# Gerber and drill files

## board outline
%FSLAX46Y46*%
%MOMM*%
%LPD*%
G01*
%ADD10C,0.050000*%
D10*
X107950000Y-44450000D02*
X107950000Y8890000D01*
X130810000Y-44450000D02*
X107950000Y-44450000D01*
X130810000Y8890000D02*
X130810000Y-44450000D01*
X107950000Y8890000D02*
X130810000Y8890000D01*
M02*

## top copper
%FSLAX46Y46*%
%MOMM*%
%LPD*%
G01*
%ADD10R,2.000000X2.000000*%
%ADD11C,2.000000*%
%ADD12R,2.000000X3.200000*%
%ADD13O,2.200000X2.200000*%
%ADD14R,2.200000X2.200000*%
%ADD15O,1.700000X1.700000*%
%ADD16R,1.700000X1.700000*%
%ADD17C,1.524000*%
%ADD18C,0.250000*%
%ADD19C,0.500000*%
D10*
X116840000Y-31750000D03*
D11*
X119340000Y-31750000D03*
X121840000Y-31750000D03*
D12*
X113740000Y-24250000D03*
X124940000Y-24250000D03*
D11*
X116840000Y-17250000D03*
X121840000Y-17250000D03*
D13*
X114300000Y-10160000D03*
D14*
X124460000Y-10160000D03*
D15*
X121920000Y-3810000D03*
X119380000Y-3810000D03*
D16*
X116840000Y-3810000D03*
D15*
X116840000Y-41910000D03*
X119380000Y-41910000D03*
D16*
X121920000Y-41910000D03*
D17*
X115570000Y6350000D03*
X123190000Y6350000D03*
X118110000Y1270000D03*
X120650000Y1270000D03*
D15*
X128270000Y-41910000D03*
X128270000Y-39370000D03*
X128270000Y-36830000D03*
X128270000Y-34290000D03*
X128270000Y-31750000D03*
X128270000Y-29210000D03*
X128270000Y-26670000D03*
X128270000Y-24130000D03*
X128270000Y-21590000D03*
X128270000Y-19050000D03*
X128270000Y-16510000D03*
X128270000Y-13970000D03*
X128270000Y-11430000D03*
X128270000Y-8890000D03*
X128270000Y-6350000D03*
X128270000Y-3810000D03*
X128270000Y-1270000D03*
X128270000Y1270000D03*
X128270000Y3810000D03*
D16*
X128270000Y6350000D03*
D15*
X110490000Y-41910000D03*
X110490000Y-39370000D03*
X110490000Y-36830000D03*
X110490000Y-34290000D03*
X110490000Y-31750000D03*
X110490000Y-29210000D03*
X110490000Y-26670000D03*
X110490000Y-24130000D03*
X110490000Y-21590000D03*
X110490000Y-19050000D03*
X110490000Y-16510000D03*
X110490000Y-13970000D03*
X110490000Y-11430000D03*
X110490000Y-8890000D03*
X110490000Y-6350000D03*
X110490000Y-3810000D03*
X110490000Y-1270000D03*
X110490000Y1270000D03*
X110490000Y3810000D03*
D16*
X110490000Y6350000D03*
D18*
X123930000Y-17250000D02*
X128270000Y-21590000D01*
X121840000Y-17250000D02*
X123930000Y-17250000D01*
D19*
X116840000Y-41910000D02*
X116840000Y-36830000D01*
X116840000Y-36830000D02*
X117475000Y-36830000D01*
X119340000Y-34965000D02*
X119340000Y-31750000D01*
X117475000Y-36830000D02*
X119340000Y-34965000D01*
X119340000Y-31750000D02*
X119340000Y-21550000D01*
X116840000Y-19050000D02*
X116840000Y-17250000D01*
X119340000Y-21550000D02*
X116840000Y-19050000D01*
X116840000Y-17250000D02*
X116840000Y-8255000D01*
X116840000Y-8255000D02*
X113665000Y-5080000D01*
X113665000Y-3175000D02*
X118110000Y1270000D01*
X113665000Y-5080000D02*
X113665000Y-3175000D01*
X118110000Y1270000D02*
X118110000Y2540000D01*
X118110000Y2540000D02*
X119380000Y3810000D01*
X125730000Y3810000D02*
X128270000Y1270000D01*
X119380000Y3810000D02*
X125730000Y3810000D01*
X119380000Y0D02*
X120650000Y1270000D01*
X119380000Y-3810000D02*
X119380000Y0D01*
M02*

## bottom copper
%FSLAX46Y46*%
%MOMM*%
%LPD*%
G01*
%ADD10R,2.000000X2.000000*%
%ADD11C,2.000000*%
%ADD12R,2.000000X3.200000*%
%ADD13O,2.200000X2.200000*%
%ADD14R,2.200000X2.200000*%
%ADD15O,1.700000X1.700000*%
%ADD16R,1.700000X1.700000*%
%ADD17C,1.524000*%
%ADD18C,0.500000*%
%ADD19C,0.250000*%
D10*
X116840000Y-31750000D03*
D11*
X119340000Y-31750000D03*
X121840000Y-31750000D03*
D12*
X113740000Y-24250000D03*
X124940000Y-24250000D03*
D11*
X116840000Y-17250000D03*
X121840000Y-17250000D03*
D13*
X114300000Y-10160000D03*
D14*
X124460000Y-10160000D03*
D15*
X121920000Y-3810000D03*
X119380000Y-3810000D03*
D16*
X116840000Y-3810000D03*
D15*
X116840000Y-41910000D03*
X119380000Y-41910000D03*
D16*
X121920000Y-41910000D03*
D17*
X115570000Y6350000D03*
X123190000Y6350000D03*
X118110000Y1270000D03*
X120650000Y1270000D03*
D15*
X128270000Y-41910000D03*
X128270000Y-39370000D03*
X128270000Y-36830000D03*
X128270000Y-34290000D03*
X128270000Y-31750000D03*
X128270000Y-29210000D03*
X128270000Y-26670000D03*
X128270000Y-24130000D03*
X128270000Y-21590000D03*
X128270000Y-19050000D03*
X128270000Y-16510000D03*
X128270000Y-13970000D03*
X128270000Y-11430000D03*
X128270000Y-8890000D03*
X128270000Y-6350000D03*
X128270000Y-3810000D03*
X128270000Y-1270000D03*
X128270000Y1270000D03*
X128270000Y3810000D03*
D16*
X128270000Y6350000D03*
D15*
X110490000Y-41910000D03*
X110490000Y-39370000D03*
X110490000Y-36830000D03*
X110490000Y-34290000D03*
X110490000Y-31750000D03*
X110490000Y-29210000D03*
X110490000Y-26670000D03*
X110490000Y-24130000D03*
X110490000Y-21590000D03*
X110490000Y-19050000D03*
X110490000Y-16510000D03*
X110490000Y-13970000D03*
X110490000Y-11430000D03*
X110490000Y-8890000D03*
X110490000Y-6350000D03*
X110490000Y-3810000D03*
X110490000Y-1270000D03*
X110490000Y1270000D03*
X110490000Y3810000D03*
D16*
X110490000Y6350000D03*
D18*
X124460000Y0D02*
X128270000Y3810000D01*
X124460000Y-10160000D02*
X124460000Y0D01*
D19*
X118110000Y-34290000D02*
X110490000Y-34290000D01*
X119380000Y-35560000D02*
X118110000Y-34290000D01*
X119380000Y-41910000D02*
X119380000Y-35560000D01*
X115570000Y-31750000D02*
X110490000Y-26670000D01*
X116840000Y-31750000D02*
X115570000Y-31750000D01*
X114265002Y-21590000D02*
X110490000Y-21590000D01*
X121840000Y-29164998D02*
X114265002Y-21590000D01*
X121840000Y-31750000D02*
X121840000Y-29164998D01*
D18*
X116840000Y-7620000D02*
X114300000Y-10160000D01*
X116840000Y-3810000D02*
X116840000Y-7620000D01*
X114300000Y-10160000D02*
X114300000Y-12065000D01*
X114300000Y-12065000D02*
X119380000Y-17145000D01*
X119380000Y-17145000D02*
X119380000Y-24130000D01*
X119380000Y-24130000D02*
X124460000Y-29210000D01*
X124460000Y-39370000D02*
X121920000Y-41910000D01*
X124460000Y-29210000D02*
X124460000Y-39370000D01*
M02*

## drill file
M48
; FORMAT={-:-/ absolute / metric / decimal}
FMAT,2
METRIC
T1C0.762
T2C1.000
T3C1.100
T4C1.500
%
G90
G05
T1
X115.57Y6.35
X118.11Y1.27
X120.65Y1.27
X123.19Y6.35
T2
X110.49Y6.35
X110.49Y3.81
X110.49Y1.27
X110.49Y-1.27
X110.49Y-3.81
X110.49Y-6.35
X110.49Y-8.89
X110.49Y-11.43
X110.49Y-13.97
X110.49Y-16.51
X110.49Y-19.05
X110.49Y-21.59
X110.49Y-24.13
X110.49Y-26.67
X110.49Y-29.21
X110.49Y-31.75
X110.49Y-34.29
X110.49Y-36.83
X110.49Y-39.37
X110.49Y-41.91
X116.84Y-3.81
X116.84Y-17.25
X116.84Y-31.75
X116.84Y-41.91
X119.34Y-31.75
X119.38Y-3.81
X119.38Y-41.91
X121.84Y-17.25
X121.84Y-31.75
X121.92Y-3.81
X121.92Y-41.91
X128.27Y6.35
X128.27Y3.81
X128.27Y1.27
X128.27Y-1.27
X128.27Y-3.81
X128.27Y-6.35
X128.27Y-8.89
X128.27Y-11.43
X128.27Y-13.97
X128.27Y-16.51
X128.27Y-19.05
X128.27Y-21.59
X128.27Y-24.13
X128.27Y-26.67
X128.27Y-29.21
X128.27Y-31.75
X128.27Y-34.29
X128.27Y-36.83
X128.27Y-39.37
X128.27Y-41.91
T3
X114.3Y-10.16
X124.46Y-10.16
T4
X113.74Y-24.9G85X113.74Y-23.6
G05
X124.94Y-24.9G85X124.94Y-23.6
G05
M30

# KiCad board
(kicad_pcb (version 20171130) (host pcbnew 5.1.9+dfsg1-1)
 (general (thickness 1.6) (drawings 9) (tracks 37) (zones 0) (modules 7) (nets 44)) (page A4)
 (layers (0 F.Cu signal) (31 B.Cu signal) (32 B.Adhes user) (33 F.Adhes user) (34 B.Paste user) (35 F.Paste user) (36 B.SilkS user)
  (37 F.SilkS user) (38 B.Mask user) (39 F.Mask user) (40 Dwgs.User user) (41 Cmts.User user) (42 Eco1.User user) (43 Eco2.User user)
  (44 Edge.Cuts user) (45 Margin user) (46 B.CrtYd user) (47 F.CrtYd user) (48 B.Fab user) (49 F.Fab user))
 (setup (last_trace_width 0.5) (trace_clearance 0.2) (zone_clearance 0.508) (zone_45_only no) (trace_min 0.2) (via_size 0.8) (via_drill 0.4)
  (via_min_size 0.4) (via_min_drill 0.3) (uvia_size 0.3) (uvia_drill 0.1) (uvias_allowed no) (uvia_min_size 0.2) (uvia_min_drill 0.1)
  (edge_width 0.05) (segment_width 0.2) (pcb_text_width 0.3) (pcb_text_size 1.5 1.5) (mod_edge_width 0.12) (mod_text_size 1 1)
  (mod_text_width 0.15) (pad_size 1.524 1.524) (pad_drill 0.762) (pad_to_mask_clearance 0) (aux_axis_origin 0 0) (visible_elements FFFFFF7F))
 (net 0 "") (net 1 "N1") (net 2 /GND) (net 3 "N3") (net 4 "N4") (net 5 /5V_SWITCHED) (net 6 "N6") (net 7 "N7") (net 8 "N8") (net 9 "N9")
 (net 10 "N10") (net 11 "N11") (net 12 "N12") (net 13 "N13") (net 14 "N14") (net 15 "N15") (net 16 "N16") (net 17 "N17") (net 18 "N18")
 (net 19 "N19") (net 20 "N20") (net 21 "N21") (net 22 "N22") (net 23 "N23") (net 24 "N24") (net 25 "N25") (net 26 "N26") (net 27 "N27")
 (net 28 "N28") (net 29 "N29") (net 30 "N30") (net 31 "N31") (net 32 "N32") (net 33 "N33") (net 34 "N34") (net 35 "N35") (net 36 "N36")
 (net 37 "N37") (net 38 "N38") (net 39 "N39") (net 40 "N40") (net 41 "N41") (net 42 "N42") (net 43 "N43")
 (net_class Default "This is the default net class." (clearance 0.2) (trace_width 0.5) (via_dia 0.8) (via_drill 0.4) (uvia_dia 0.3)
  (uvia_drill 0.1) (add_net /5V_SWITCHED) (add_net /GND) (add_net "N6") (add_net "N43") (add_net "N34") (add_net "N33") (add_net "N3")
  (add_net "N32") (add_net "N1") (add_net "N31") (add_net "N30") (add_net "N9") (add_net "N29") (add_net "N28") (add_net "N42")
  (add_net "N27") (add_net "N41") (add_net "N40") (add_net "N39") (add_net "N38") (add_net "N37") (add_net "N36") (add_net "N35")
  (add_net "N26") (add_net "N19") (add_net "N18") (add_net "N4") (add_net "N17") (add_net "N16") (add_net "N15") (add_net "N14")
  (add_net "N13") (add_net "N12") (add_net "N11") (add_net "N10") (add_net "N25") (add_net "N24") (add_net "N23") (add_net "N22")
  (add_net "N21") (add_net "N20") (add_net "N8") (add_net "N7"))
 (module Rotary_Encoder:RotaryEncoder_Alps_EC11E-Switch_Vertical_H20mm (layer F.Cu) (at 116.84 31.75 90)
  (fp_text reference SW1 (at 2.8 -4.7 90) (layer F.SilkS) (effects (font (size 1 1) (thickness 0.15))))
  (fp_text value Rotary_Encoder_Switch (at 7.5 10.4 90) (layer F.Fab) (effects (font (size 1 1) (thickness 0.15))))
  (pad A thru_hole rect (at 0 0 90) (size 2 2) (drill 1) (layers *.Cu *.Mask) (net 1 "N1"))
  (pad C thru_hole circle (at 0 2.5 90) (size 2 2) (drill 1) (layers *.Cu *.Mask) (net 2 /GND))
  (pad B thru_hole circle (at 0 5 90) (size 2 2) (drill 1) (layers *.Cu *.Mask) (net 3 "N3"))
  (pad MP thru_hole rect (at 7.5 -3.1 90) (size 3.2 2) (drill oval 2.8 1.5) (layers *.Cu *.Mask))
  (pad MP thru_hole rect (at 7.5 8.1 90) (size 3.2 2) (drill oval 2.8 1.5) (layers *.Cu *.Mask))
  (pad S2 thru_hole circle (at 14.5 0 90) (size 2 2) (drill 1) (layers *.Cu *.Mask) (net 2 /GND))
  (pad S1 thru_hole circle (at 14.5 5 90) (size 2 2) (drill 1) (layers *.Cu *.Mask) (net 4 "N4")))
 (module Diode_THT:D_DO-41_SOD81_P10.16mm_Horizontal (layer F.Cu) (at 124.46 10.16 180)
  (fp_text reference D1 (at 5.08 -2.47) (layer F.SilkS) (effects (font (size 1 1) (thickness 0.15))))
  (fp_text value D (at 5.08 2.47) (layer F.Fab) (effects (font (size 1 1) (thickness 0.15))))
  (pad 2 thru_hole oval (at 10.16 0 180) (size 2.2 2.2) (drill 1.1) (layers *.Cu *.Mask) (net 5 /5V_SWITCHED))
  (pad 1 thru_hole rect (at 0 0 180) (size 2.2 2.2) (drill 1.1) (layers *.Cu *.Mask) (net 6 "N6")))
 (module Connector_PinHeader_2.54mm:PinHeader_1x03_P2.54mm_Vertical (layer F.Cu) (at 116.84 3.81 90)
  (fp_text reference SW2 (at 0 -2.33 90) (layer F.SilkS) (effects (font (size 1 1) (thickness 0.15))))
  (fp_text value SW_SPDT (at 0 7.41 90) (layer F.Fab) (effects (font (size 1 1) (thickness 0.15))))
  (pad 3 thru_hole oval (at 0 5.08 90) (size 1.7 1.7) (drill 1) (layers *.Cu *.Mask) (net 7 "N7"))
  (pad 2 thru_hole oval (at 0 2.54 90) (size 1.7 1.7) (drill 1) (layers *.Cu *.Mask) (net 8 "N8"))
  (pad 1 thru_hole rect (at 0 0 90) (size 1.7 1.7) (drill 1) (layers *.Cu *.Mask) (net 5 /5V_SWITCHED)))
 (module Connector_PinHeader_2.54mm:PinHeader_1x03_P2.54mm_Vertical (layer F.Cu) (at 121.92 41.91 270)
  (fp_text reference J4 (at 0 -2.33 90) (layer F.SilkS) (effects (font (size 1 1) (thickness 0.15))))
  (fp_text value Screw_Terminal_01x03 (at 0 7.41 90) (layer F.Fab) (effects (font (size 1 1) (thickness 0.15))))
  (pad 3 thru_hole oval (at 0 5.08 270) (size 1.7 1.7) (drill 1) (layers *.Cu *.Mask) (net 2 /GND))
  (pad 2 thru_hole oval (at 0 2.54 270) (size 1.7 1.7) (drill 1) (layers *.Cu *.Mask) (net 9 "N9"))
  (pad 1 thru_hole rect (at 0 0 270) (size 1.7 1.7) (drill 1) (layers *.Cu *.Mask) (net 5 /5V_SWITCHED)))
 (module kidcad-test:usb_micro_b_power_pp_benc (layer F.Cu) (at 124.46 -3.81 180)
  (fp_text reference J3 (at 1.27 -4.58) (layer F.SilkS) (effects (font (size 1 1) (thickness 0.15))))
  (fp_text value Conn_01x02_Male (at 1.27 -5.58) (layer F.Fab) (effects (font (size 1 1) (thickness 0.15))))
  (pad 3 thru_hole circle (at 8.89 2.54 180) (size 1.524 1.524) (drill 0.762) (layers *.Cu *.Mask))
  (pad 4 thru_hole circle (at 1.27 2.54 180) (size 1.524 1.524) (drill 0.762) (layers *.Cu *.Mask))
  (pad 1 thru_hole circle (at 6.35 -2.54 180) (size 1.524 1.524) (drill 0.762) (layers *.Cu *.Mask) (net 2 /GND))
  (pad 2 thru_hole circle (at 3.81 -2.54 180) (size 1.524 1.524) (drill 0.762) (layers *.Cu *.Mask) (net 8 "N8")))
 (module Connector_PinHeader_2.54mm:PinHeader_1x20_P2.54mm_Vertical (layer F.Cu) (at 128.27 -6.35)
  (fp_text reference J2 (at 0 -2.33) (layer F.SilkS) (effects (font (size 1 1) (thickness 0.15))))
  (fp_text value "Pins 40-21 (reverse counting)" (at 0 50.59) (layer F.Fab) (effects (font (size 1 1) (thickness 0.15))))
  (pad 20 thru_hole oval (at 0 48.26) (size 1.7 1.7) (drill 1) (layers *.Cu *.Mask) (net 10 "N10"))
  (pad 19 thru_hole oval (at 0 45.72) (size 1.7 1.7) (drill 1) (layers *.Cu *.Mask) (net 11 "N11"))
  (pad 18 thru_hole oval (at 0 43.18) (size 1.7 1.7) (drill 1) (layers *.Cu *.Mask) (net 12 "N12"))
  (pad 17 thru_hole oval (at 0 40.64) (size 1.7 1.7) (drill 1) (layers *.Cu *.Mask) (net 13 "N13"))
  (pad 16 thru_hole oval (at 0 38.1) (size 1.7 1.7) (drill 1) (layers *.Cu *.Mask) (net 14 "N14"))
  (pad 15 thru_hole oval (at 0 35.56) (size 1.7 1.7) (drill 1) (layers *.Cu *.Mask) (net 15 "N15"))
  (pad 14 thru_hole oval (at 0 33.02) (size 1.7 1.7) (drill 1) (layers *.Cu *.Mask) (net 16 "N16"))
  (pad 13 thru_hole oval (at 0 30.48) (size 1.7 1.7) (drill 1) (layers *.Cu *.Mask) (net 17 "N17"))
  (pad 12 thru_hole oval (at 0 27.94) (size 1.7 1.7) (drill 1) (layers *.Cu *.Mask) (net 4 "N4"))
  (pad 11 thru_hole oval (at 0 25.4) (size 1.7 1.7) (drill 1) (layers *.Cu *.Mask) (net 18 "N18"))
  (pad 10 thru_hole oval (at 0 22.86) (size 1.7 1.7) (drill 1) (layers *.Cu *.Mask) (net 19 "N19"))
  (pad 9 thru_hole oval (at 0 20.32) (size 1.7 1.7) (drill 1) (layers *.Cu *.Mask) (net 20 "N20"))
  (pad 8 thru_hole oval (at 0 17.78) (size 1.7 1.7) (drill 1) (layers *.Cu *.Mask) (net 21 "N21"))
  (pad 7 thru_hole oval (at 0 15.24) (size 1.7 1.7) (drill 1) (layers *.Cu *.Mask) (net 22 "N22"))
  (pad 6 thru_hole oval (at 0 12.7) (size 1.7 1.7) (drill 1) (layers *.Cu *.Mask) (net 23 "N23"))
  (pad 5 thru_hole oval (at 0 10.16) (size 1.7 1.7) (drill 1) (layers *.Cu *.Mask) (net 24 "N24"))
  (pad 4 thru_hole oval (at 0 7.62) (size 1.7 1.7) (drill 1) (layers *.Cu *.Mask) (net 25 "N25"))
  (pad 3 thru_hole oval (at 0 5.08) (size 1.7 1.7) (drill 1) (layers *.Cu *.Mask) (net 2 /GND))
  (pad 2 thru_hole oval (at 0 2.54) (size 1.7 1.7) (drill 1) (layers *.Cu *.Mask) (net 6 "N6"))
  (pad 1 thru_hole rect (at 0 0) (size 1.7 1.7) (drill 1) (layers *.Cu *.Mask) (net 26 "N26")))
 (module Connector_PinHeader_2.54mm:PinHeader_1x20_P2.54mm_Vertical (layer F.Cu) (at 110.49 -6.35)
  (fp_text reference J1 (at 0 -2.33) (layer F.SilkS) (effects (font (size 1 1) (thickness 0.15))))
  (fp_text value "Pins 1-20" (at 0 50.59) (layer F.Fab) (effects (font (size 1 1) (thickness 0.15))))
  (pad 20 thru_hole oval (at 0 48.26) (size 1.7 1.7) (drill 1) (layers *.Cu *.Mask) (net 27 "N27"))
  (pad 19 thru_hole oval (at 0 45.72) (size 1.7 1.7) (drill 1) (layers *.Cu *.Mask) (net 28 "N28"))
  (pad 18 thru_hole oval (at 0 43.18) (size 1.7 1.7) (drill 1) (layers *.Cu *.Mask) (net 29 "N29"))
  (pad 17 thru_hole oval (at 0 40.64) (size 1.7 1.7) (drill 1) (layers *.Cu *.Mask) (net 9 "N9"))
  (pad 16 thru_hole oval (at 0 38.1) (size 1.7 1.7) (drill 1) (layers *.Cu *.Mask) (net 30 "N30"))
  (pad 15 thru_hole oval (at 0 35.56) (size 1.7 1.7) (drill 1) (layers *.Cu *.Mask) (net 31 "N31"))
  (pad 14 thru_hole oval (at 0 33.02) (size 1.7 1.7) (drill 1) (layers *.Cu *.Mask) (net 1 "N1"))
  (pad 13 thru_hole oval (at 0 30.48) (size 1.7 1.7) (drill 1) (layers *.Cu *.Mask) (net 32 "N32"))
  (pad 12 thru_hole oval (at 0 27.94) (size 1.7 1.7) (drill 1) (layers *.Cu *.Mask) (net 3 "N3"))
  (pad 11 thru_hole oval (at 0 25.4) (size 1.7 1.7) (drill 1) (layers *.Cu *.Mask) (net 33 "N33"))
  (pad 10 thru_hole oval (at 0 22.86) (size 1.7 1.7) (drill 1) (layers *.Cu *.Mask) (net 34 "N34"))
  (pad 9 thru_hole oval (at 0 20.32) (size 1.7 1.7) (drill 1) (layers *.Cu *.Mask) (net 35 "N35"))
  (pad 8 thru_hole oval (at 0 17.78) (size 1.7 1.7) (drill 1) (layers *.Cu *.Mask) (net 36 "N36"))
  (pad 7 thru_hole oval (at 0 15.24) (size 1.7 1.7) (drill 1) (layers *.Cu *.Mask) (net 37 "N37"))
  (pad 6 thru_hole oval (at 0 12.7) (size 1.7 1.7) (drill 1) (layers *.Cu *.Mask) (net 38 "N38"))
  (pad 5 thru_hole oval (at 0 10.16) (size 1.7 1.7) (drill 1) (layers *.Cu *.Mask) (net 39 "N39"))
  (pad 4 thru_hole oval (at 0 7.62) (size 1.7 1.7) (drill 1) (layers *.Cu *.Mask) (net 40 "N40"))
  (pad 3 thru_hole oval (at 0 5.08) (size 1.7 1.7) (drill 1) (layers *.Cu *.Mask) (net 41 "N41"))
  (pad 2 thru_hole oval (at 0 2.54) (size 1.7 1.7) (drill 1) (layers *.Cu *.Mask) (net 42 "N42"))
  (pad 1 thru_hole rect (at 0 0) (size 1.7 1.7) (drill 1) (layers *.Cu *.Mask) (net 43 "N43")))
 (gr_line (start 107.95 44.45) (end 107.95 -8.89) (layer Edge.Cuts) (width 0.05))
 (gr_line (start 130.81 44.45) (end 107.95 44.45) (layer Edge.Cuts) (width 0.05))
 (gr_line (start 130.81 -8.89) (end 130.81 44.45) (layer Edge.Cuts) (width 0.05))
 (gr_line (start 107.95 -8.89) (end 130.81 -8.89) (layer Edge.Cuts) (width 0.05))
 (segment (start 124.46 0) (end 128.27 -3.81) (width 0.5) (layer B.Cu) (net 6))
 (segment (start 124.46 10.16) (end 124.46 0) (width 0.5) (layer B.Cu) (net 6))
 (segment (start 118.11 34.29) (end 110.49 34.29) (width 0.25) (layer B.Cu) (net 9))
 (segment (start 119.38 35.56) (end 118.11 34.29) (width 0.25) (layer B.Cu) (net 9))
 (segment (start 119.38 41.91) (end 119.38 35.56) (width 0.25) (layer B.Cu) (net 9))
 (segment (start 115.57 31.75) (end 110.49 26.67) (width 0.25) (layer B.Cu) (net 1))
 (segment (start 116.84 31.75) (end 115.57 31.75) (width 0.25) (layer B.Cu) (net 1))
 (segment (start 114.265002 21.59) (end 110.49 21.59) (width 0.25) (layer B.Cu) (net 3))
 (segment (start 121.84 29.164998) (end 114.265002 21.59) (width 0.25) (layer B.Cu) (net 3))
 (segment (start 121.84 31.75) (end 121.84 29.164998) (width 0.25) (layer B.Cu) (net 3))
 (segment (start 123.93 17.25) (end 128.27 21.59) (width 0.25) (layer F.Cu) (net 4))
 (segment (start 121.84 17.25) (end 123.93 17.25) (width 0.25) (layer F.Cu) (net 4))
 (segment (start 116.84 41.91) (end 116.84 36.83) (width 0.5) (layer F.Cu) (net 2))
 (segment (start 116.84 36.83) (end 117.475 36.83) (width 0.5) (layer F.Cu) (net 2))
 (segment (start 119.34 34.965) (end 119.34 31.75) (width 0.5) (layer F.Cu) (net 2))
 (segment (start 117.475 36.83) (end 119.34 34.965) (width 0.5) (layer F.Cu) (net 2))
 (segment (start 119.34 31.75) (end 119.34 21.55) (width 0.5) (layer F.Cu) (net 2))
 (segment (start 116.84 19.05) (end 116.84 17.25) (width 0.5) (layer F.Cu) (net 2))
 (segment (start 119.34 21.55) (end 116.84 19.05) (width 0.5) (layer F.Cu) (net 2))
 (segment (start 116.84 17.25) (end 116.84 8.255) (width 0.5) (layer F.Cu) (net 2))
 (segment (start 116.84 8.255) (end 113.665 5.08) (width 0.5) (layer F.Cu) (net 2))
 (segment (start 113.665 3.175) (end 118.11 -1.27) (width 0.5) (layer F.Cu) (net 2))
 (segment (start 113.665 5.08) (end 113.665 3.175) (width 0.5) (layer F.Cu) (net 2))
 (segment (start 118.11 -1.27) (end 118.11 -2.54) (width 0.5) (layer F.Cu) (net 2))
 (segment (start 118.11 -2.54) (end 119.38 -3.81) (width 0.5) (layer F.Cu) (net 2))
 (segment (start 125.73 -3.81) (end 128.27 -1.27) (width 0.5) (layer F.Cu) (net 2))
 (segment (start 119.38 -3.81) (end 125.73 -3.81) (width 0.5) (layer F.Cu) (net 2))
 (segment (start 119.38 0) (end 120.65 -1.27) (width 0.5) (layer F.Cu) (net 8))
 (segment (start 119.38 3.81) (end 119.38 0) (width 0.5) (layer F.Cu) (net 8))
 (segment (start 116.84 7.62) (end 114.3 10.16) (width 0.5) (layer B.Cu) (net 5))
 (segment (start 116.84 3.81) (end 116.84 7.62) (width 0.5) (layer B.Cu) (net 5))
 (segment (start 114.3 10.16) (end 114.3 12.065) (width 0.5) (layer B.Cu) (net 5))
 (segment (start 114.3 12.065) (end 119.38 17.145) (width 0.5) (layer B.Cu) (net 5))
 (segment (start 119.38 17.145) (end 119.38 24.13) (width 0.5) (layer B.Cu) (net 5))
 (segment (start 119.38 24.13) (end 124.46 29.21) (width 0.5) (layer B.Cu) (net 5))
 (segment (start 124.46 39.37) (end 121.92 41.91) (width 0.5) (layer B.Cu) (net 5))
 (segment (start 124.46 29.21) (end 124.46 39.37) (width 0.5) (layer B.Cu) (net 5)))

